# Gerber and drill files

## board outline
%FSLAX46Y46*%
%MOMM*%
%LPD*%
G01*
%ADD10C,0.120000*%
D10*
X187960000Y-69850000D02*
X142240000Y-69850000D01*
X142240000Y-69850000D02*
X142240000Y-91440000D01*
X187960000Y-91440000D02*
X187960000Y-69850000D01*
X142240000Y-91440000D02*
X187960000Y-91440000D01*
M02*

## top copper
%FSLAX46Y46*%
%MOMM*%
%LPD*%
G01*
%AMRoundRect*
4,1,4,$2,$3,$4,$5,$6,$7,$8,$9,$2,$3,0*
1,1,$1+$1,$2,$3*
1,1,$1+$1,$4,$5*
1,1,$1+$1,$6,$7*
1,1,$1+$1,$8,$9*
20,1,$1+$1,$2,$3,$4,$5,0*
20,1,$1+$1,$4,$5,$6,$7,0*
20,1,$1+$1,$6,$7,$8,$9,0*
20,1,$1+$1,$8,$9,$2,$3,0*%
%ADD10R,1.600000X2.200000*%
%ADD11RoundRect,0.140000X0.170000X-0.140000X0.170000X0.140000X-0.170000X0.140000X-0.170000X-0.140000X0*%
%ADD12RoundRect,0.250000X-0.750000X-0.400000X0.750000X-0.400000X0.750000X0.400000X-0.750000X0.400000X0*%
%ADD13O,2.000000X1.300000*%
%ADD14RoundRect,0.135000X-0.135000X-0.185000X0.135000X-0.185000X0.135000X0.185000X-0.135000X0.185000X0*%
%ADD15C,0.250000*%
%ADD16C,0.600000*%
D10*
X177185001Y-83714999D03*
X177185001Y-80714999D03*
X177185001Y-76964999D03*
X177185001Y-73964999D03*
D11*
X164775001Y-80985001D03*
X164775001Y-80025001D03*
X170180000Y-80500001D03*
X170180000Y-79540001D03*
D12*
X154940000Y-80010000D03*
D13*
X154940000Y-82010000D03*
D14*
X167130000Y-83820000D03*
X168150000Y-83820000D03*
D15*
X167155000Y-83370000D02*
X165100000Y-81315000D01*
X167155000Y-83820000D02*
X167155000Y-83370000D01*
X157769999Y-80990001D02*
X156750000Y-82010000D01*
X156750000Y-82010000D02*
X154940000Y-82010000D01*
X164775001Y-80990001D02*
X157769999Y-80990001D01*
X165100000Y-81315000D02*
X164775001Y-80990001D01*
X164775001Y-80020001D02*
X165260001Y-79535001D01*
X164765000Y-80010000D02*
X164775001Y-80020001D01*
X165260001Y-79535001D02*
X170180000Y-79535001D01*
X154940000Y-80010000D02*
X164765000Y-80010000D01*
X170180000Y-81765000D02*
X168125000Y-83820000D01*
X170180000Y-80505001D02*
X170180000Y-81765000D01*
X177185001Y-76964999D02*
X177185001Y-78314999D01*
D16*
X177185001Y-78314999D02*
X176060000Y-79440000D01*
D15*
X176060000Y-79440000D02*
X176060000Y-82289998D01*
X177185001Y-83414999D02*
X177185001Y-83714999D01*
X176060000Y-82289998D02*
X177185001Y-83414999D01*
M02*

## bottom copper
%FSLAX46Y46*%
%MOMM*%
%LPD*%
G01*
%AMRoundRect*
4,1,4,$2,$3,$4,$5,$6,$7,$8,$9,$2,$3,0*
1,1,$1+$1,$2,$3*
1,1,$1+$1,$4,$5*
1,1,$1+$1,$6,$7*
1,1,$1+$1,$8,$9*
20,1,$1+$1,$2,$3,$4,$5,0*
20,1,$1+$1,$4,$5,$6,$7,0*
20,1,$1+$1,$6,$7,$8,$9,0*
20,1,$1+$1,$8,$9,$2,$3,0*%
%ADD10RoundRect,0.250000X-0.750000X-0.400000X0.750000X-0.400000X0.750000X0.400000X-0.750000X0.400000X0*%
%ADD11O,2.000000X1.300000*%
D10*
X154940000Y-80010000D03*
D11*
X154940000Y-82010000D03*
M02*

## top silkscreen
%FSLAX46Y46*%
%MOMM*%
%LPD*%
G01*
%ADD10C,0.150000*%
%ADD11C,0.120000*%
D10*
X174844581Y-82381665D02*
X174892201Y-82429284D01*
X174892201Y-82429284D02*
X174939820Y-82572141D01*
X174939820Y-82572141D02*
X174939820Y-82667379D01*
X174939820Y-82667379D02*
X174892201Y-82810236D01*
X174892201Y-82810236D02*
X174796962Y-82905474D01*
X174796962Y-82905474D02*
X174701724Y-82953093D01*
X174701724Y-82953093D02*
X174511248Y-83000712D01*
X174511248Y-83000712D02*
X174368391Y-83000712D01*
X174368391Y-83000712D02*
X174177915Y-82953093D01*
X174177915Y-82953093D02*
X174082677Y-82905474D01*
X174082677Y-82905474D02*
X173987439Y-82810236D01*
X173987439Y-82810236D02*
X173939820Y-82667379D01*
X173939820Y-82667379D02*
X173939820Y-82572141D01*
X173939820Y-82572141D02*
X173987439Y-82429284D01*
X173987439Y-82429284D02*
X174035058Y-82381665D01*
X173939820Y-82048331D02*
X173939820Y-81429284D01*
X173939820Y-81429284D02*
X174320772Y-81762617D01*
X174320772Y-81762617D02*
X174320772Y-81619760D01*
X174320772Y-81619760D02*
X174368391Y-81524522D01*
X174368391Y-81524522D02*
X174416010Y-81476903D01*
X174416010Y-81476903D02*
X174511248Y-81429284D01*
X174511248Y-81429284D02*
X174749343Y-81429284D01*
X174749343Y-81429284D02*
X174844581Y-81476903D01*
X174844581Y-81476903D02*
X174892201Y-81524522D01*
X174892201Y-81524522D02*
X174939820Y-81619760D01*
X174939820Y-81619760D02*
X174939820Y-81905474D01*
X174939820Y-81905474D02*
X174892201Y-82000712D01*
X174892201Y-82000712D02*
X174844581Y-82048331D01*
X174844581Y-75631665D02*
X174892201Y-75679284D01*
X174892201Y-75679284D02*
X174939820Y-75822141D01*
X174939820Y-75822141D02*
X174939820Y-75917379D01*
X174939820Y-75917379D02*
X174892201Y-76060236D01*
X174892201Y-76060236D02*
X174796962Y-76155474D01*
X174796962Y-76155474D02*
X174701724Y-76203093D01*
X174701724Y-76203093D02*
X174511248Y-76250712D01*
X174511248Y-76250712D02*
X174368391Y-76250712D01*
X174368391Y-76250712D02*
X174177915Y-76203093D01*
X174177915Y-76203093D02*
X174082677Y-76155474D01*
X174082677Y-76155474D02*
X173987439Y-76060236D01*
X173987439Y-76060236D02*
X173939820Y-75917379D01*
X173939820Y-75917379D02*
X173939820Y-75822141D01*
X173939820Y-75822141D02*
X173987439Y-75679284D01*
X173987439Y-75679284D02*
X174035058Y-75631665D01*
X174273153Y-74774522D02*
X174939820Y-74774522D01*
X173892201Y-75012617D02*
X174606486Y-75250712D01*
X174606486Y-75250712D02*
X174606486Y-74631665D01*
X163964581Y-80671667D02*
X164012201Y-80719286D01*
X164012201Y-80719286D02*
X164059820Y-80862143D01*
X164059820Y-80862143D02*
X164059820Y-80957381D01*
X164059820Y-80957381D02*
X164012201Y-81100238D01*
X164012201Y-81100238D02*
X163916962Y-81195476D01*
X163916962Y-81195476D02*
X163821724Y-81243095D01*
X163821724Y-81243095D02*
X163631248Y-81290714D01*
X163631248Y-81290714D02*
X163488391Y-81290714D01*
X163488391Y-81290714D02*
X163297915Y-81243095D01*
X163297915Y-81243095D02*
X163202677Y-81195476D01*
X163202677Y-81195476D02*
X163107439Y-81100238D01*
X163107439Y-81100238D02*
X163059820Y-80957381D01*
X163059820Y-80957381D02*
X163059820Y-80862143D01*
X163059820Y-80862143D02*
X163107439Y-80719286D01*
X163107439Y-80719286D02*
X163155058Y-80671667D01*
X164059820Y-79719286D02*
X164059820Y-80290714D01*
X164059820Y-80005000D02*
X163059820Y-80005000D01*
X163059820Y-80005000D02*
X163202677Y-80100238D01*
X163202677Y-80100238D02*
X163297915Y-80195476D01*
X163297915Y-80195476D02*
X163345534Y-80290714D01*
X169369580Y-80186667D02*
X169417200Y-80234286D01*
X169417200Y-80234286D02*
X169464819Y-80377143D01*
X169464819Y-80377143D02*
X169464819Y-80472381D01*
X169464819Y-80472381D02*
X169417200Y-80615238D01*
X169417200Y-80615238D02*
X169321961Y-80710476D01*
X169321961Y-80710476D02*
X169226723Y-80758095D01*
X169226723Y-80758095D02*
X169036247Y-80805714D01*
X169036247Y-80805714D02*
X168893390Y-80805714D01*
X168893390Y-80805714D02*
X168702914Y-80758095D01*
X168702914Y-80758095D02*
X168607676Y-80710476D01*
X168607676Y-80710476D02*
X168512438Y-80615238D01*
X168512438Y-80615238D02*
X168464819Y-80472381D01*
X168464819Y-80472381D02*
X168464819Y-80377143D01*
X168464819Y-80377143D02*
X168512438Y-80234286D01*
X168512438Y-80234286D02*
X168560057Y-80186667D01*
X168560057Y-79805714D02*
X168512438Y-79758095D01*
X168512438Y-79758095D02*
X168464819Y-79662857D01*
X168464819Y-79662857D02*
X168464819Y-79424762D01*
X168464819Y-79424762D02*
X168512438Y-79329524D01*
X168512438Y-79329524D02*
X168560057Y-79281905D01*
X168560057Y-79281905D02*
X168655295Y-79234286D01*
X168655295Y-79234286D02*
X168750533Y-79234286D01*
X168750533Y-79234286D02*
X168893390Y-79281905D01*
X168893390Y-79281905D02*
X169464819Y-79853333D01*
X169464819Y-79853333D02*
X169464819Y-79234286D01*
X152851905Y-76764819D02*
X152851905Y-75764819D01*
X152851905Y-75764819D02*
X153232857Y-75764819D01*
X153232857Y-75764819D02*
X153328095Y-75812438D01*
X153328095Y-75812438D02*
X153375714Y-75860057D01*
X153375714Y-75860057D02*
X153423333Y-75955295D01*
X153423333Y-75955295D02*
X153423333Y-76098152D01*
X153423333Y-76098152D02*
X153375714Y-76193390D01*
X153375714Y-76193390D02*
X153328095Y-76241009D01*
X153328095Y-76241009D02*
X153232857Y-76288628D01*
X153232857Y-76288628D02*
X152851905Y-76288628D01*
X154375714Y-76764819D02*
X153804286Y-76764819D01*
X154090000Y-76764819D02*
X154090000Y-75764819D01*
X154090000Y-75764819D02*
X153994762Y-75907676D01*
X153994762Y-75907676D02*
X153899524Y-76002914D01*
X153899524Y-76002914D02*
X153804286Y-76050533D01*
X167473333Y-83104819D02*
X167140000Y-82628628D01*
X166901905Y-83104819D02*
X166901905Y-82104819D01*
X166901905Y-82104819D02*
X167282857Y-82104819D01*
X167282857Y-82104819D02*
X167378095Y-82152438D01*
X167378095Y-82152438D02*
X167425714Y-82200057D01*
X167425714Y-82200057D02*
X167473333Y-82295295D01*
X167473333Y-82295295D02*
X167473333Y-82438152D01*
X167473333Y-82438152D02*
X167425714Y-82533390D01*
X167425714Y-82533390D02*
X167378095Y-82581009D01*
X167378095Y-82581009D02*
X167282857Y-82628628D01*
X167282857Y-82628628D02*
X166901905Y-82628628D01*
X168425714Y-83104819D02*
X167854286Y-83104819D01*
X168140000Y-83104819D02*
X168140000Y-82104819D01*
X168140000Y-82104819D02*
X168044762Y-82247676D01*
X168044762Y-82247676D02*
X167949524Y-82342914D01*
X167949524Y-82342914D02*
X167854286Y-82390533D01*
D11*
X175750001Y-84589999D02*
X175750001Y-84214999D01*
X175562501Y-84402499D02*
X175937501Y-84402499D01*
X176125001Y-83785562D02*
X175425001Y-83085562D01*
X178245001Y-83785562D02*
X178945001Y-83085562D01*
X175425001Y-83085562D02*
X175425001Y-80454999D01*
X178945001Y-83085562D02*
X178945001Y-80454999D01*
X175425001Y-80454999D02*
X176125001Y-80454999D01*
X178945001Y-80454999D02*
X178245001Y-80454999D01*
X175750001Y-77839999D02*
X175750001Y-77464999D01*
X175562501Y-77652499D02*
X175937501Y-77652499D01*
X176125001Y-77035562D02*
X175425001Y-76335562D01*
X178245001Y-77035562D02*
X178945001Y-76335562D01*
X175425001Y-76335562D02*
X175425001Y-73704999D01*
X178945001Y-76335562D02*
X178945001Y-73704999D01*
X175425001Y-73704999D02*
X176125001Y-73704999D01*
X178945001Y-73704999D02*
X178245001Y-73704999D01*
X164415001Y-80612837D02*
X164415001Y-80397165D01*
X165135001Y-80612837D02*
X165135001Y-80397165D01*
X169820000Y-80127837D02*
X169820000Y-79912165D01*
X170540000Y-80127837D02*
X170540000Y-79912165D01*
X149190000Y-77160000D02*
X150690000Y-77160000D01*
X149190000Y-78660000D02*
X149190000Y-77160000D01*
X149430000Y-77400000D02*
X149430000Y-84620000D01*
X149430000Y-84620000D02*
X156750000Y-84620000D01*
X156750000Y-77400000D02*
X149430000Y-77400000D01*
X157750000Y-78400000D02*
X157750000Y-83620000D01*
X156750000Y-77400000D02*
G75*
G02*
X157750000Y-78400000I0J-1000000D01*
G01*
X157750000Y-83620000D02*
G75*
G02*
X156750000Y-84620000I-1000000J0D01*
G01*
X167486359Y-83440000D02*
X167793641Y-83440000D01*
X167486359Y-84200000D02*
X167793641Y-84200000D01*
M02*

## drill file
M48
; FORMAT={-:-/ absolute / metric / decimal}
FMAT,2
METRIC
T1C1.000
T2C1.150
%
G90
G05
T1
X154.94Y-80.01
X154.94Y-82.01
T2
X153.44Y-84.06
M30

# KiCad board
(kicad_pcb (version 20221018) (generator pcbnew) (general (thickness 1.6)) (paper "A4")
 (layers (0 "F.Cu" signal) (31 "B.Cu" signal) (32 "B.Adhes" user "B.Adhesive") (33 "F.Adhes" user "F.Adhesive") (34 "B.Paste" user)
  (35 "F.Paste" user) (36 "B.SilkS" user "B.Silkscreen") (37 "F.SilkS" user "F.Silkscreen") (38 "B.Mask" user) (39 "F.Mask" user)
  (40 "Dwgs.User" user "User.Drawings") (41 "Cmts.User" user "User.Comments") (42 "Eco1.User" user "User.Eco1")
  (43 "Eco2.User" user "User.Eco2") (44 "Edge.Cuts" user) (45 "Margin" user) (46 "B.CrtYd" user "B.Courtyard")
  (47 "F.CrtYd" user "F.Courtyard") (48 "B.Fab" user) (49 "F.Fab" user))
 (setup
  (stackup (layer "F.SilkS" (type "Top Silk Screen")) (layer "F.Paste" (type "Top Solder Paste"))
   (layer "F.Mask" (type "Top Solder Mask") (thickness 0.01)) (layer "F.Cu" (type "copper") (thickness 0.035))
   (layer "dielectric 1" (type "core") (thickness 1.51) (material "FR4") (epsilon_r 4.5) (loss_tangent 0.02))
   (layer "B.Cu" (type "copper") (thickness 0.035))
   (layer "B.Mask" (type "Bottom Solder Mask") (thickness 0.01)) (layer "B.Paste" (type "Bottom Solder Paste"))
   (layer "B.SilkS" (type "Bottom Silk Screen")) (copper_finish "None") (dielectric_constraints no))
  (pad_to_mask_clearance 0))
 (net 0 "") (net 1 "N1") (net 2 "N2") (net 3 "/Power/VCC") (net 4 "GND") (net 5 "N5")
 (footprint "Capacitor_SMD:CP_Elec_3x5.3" (layer "F.Cu") (at 177.185001 82.214999 90)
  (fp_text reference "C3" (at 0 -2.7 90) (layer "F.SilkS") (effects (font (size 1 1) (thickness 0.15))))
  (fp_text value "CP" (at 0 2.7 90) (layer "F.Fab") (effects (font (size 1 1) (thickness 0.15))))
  (fp_line (start -2.375 -1.435) (end -2 -1.435) (stroke (width 0.12) (type solid)) (layer "F.SilkS"))
  (fp_line (start -2.1875 -1.6225) (end -2.1875 -1.2475) (stroke (width 0.12) (type solid)) (layer "F.SilkS"))
  (fp_line (start -1.570563 -1.06) (end -0.870563 -1.76) (stroke (width 0.12) (type solid)) (layer "F.SilkS"))
  (fp_line (start -1.570563 1.06) (end -0.870563 1.76) (stroke (width 0.12) (type solid)) (layer "F.SilkS"))
  (fp_line (start -0.870563 -1.76) (end 1.76 -1.76) (stroke (width 0.12) (type solid)) (layer "F.SilkS"))
  (fp_line (start -0.870563 1.76) (end 1.76 1.76) (stroke (width 0.12) (type solid)) (layer "F.SilkS"))
  (fp_line (start 1.76 -1.76) (end 1.76 -1.06) (stroke (width 0.12) (type solid)) (layer "F.SilkS"))
  (fp_line (start 1.76 1.76) (end 1.76 1.06) (stroke (width 0.12) (type solid)) (layer "F.SilkS"))
  (pad "1" smd rect (at -1.5 0 90) (size 2.2 1.6) (layers "F.Cu" "F.Paste" "F.Mask") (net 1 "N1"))
  (pad "2" smd rect (at 1.5 0 90) (size 2.2 1.6) (layers "F.Cu" "F.Paste" "F.Mask") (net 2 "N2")))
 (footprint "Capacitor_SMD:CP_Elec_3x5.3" (layer "F.Cu") (at 177.185001 75.464999 90)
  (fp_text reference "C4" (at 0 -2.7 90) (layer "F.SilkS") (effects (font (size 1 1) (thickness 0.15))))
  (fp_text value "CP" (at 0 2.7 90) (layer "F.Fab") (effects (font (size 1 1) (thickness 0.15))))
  (fp_line (start -2.375 -1.435) (end -2 -1.435) (stroke (width 0.12) (type solid)) (layer "F.SilkS"))
  (fp_line (start -2.1875 -1.6225) (end -2.1875 -1.2475) (stroke (width 0.12) (type solid)) (layer "F.SilkS"))
  (fp_line (start -1.570563 -1.06) (end -0.870563 -1.76) (stroke (width 0.12) (type solid)) (layer "F.SilkS"))
  (fp_line (start -1.570563 1.06) (end -0.870563 1.76) (stroke (width 0.12) (type solid)) (layer "F.SilkS"))
  (fp_line (start -0.870563 -1.76) (end 1.76 -1.76) (stroke (width 0.12) (type solid)) (layer "F.SilkS"))
  (fp_line (start -0.870563 1.76) (end 1.76 1.76) (stroke (width 0.12) (type solid)) (layer "F.SilkS"))
  (fp_line (start 1.76 -1.76) (end 1.76 -1.06) (stroke (width 0.12) (type solid)) (layer "F.SilkS"))
  (fp_line (start 1.76 1.76) (end 1.76 1.06) (stroke (width 0.12) (type solid)) (layer "F.SilkS"))
  (pad "1" smd rect (at -1.5 0 90) (size 2.2 1.6) (layers "F.Cu" "F.Paste" "F.Mask") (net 1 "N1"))
  (pad "2" smd rect (at 1.5 0 90) (size 2.2 1.6) (layers "F.Cu" "F.Paste" "F.Mask") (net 2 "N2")))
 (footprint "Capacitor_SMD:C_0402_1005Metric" (layer "F.Cu") (at 164.775001 80.505001 90)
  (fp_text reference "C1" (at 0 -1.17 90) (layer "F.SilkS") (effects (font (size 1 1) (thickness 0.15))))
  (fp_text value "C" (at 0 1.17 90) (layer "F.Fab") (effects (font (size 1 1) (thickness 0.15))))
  (fp_line (start -0.107836 -0.36) (end 0.107836 -0.36) (stroke (width 0.12) (type solid)) (layer "F.SilkS"))
  (fp_line (start -0.107836 0.36) (end 0.107836 0.36) (stroke (width 0.12) (type solid)) (layer "F.SilkS"))
  (pad "1" smd roundrect (at -0.48 0 90) (size 0.56 0.62) (layers "F.Cu" "F.Paste" "F.Mask") (roundrect_rratio 0.25) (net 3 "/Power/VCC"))
  (pad "2" smd roundrect (at 0.48 0 90) (size 0.56 0.62) (layers "F.Cu" "F.Paste" "F.Mask") (roundrect_rratio 0.25) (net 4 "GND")))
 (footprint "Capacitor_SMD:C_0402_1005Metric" (layer "F.Cu") (at 170.18 80.020001 90)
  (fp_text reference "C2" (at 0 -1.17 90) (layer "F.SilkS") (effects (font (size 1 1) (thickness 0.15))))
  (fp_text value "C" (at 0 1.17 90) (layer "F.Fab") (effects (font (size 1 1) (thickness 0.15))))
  (fp_line (start -0.107836 -0.36) (end 0.107836 -0.36) (stroke (width 0.12) (type solid)) (layer "F.SilkS"))
  (fp_line (start -0.107836 0.36) (end 0.107836 0.36) (stroke (width 0.12) (type solid)) (layer "F.SilkS"))
  (pad "1" smd roundrect (at -0.48 0 90) (size 0.56 0.62) (layers "F.Cu" "F.Paste" "F.Mask") (roundrect_rratio 0.25) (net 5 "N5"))
  (pad "2" smd roundrect (at 0.48 0 90) (size 0.56 0.62) (layers "F.Cu" "F.Paste" "F.Mask") (roundrect_rratio 0.25) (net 4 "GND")))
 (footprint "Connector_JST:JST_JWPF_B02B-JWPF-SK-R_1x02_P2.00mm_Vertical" (layer "F.Cu") (at 154.94 80.01)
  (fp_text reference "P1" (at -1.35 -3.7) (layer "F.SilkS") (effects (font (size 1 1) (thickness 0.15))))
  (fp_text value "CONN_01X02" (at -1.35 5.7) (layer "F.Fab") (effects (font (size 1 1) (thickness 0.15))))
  (fp_line (start -5.75 -2.85) (end -4.25 -2.85) (stroke (width 0.12) (type solid)) (layer "F.SilkS"))
  (fp_line (start -5.75 -1.35) (end -5.75 -2.85) (stroke (width 0.12) (type solid)) (layer "F.SilkS"))
  (fp_line (start -5.51 -2.61) (end -5.51 4.61) (stroke (width 0.12) (type solid)) (layer "F.SilkS"))
  (fp_line (start -5.51 4.61) (end 1.81 4.61) (stroke (width 0.12) (type solid)) (layer "F.SilkS"))
  (fp_line (start 1.81 -2.61) (end -5.51 -2.61) (stroke (width 0.12) (type solid)) (layer "F.SilkS"))
  (fp_line (start 2.81 -1.61) (end 2.81 3.61) (stroke (width 0.12) (type solid)) (layer "F.SilkS"))
  (fp_arc (start 1.81 -2.61) (mid 2.517107 -2.317107) (end 2.81 -1.61) (stroke (width 0.12) (type solid)) (layer "F.SilkS"))
  (fp_arc (start 2.81 3.61) (mid 2.517107 4.317107) (end 1.81 4.61) (stroke (width 0.12) (type solid)) (layer "F.SilkS"))
  (pad "" np_thru_hole circle (at -1.5 4.05) (size 1.15 1.15) (drill 1.15) (layers "*.Cu" "*.Mask"))
  (pad "1" thru_hole roundrect (at 0 0) (size 2 1.3) (drill 1) (layers "*.Cu" "*.Mask") (roundrect_rratio 0.192308) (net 4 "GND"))
  (pad "2" thru_hole oval (at 0 2) (size 2 1.3) (drill 1) (layers "*.Cu" "*.Mask") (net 3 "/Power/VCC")))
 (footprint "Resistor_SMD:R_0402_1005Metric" (layer "F.Cu") (at 167.64 83.82)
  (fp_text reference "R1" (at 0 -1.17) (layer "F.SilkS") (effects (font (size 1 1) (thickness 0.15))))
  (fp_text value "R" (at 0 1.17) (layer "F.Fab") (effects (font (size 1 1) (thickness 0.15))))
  (fp_line (start -0.153641 -0.38) (end 0.153641 -0.38) (stroke (width 0.12) (type solid)) (layer "F.SilkS"))
  (fp_line (start -0.153641 0.38) (end 0.153641 0.38) (stroke (width 0.12) (type solid)) (layer "F.SilkS"))
  (pad "1" smd roundrect (at -0.51 0) (size 0.54 0.64) (layers "F.Cu" "F.Paste" "F.Mask") (roundrect_rratio 0.25) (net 3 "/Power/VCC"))
  (pad "2" smd roundrect (at 0.51 0) (size 0.54 0.64) (layers "F.Cu" "F.Paste" "F.Mask") (roundrect_rratio 0.25) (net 5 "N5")))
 (gr_line (start 187.96 69.85) (end 142.24 69.85) (stroke (width 0.12) (type solid)) (layer "Edge.Cuts"))
 (gr_line (start 142.24 69.85) (end 142.24 91.44) (stroke (width 0.12) (type solid)) (layer "Edge.Cuts"))
 (gr_line (start 187.96 91.44) (end 187.96 69.85) (stroke (width 0.12) (type solid)) (layer "Edge.Cuts"))
 (gr_line (start 142.24 91.44) (end 187.96 91.44) (stroke (width 0.12) (type solid)) (layer "Edge.Cuts"))
 (segment (start 167.155 83.37) (end 165.1 81.315) (width 0.25) (layer "F.Cu") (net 3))
 (segment (start 167.155 83.82) (end 167.155 83.37) (width 0.25) (layer "F.Cu") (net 3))
 (segment (start 157.769999 80.990001) (end 156.75 82.01) (width 0.25) (layer "F.Cu") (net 3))
 (segment (start 156.75 82.01) (end 154.94 82.01) (width 0.25) (layer "F.Cu") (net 3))
 (segment (start 164.775001 80.990001) (end 157.769999 80.990001) (width 0.25) (layer "F.Cu") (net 3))
 (segment (start 165.1 81.315) (end 164.775001 80.990001) (width 0.25) (layer "F.Cu") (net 3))
 (segment (start 164.775001 80.020001) (end 165.260001 79.535001) (width 0.25) (layer "F.Cu") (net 4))
 (segment (start 164.765 80.01) (end 164.775001 80.020001) (width 0.25) (layer "F.Cu") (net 4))
 (segment (start 165.260001 79.535001) (end 170.18 79.535001) (width 0.25) (layer "F.Cu") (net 4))
 (segment (start 154.94 80.01) (end 164.765 80.01) (width 0.25) (layer "F.Cu") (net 4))
 (segment (start 170.18 81.765) (end 168.125 83.82) (width 0.25) (layer "F.Cu") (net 5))
 (segment (start 170.18 80.505001) (end 170.18 81.765) (width 0.25) (layer "F.Cu") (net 5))
 (segment (start 177.185001 76.964999) (end 177.185001 78.314999) (width 0.25) (layer "F.Cu") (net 1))
 (segment (start 177.185001 78.314999) (end 176.06 79.44) (width 0.6) (layer "F.Cu") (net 1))
 (segment (start 176.06 79.44) (end 176.06 82.289998) (width 0.25) (layer "F.Cu") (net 1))
 (segment (start 177.185001 83.414999) (end 177.185001 83.714999) (width 0.25) (layer "F.Cu") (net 1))
 (segment (start 176.06 82.289998) (end 177.185001 83.414999) (width 0.25) (layer "F.Cu") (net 1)))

